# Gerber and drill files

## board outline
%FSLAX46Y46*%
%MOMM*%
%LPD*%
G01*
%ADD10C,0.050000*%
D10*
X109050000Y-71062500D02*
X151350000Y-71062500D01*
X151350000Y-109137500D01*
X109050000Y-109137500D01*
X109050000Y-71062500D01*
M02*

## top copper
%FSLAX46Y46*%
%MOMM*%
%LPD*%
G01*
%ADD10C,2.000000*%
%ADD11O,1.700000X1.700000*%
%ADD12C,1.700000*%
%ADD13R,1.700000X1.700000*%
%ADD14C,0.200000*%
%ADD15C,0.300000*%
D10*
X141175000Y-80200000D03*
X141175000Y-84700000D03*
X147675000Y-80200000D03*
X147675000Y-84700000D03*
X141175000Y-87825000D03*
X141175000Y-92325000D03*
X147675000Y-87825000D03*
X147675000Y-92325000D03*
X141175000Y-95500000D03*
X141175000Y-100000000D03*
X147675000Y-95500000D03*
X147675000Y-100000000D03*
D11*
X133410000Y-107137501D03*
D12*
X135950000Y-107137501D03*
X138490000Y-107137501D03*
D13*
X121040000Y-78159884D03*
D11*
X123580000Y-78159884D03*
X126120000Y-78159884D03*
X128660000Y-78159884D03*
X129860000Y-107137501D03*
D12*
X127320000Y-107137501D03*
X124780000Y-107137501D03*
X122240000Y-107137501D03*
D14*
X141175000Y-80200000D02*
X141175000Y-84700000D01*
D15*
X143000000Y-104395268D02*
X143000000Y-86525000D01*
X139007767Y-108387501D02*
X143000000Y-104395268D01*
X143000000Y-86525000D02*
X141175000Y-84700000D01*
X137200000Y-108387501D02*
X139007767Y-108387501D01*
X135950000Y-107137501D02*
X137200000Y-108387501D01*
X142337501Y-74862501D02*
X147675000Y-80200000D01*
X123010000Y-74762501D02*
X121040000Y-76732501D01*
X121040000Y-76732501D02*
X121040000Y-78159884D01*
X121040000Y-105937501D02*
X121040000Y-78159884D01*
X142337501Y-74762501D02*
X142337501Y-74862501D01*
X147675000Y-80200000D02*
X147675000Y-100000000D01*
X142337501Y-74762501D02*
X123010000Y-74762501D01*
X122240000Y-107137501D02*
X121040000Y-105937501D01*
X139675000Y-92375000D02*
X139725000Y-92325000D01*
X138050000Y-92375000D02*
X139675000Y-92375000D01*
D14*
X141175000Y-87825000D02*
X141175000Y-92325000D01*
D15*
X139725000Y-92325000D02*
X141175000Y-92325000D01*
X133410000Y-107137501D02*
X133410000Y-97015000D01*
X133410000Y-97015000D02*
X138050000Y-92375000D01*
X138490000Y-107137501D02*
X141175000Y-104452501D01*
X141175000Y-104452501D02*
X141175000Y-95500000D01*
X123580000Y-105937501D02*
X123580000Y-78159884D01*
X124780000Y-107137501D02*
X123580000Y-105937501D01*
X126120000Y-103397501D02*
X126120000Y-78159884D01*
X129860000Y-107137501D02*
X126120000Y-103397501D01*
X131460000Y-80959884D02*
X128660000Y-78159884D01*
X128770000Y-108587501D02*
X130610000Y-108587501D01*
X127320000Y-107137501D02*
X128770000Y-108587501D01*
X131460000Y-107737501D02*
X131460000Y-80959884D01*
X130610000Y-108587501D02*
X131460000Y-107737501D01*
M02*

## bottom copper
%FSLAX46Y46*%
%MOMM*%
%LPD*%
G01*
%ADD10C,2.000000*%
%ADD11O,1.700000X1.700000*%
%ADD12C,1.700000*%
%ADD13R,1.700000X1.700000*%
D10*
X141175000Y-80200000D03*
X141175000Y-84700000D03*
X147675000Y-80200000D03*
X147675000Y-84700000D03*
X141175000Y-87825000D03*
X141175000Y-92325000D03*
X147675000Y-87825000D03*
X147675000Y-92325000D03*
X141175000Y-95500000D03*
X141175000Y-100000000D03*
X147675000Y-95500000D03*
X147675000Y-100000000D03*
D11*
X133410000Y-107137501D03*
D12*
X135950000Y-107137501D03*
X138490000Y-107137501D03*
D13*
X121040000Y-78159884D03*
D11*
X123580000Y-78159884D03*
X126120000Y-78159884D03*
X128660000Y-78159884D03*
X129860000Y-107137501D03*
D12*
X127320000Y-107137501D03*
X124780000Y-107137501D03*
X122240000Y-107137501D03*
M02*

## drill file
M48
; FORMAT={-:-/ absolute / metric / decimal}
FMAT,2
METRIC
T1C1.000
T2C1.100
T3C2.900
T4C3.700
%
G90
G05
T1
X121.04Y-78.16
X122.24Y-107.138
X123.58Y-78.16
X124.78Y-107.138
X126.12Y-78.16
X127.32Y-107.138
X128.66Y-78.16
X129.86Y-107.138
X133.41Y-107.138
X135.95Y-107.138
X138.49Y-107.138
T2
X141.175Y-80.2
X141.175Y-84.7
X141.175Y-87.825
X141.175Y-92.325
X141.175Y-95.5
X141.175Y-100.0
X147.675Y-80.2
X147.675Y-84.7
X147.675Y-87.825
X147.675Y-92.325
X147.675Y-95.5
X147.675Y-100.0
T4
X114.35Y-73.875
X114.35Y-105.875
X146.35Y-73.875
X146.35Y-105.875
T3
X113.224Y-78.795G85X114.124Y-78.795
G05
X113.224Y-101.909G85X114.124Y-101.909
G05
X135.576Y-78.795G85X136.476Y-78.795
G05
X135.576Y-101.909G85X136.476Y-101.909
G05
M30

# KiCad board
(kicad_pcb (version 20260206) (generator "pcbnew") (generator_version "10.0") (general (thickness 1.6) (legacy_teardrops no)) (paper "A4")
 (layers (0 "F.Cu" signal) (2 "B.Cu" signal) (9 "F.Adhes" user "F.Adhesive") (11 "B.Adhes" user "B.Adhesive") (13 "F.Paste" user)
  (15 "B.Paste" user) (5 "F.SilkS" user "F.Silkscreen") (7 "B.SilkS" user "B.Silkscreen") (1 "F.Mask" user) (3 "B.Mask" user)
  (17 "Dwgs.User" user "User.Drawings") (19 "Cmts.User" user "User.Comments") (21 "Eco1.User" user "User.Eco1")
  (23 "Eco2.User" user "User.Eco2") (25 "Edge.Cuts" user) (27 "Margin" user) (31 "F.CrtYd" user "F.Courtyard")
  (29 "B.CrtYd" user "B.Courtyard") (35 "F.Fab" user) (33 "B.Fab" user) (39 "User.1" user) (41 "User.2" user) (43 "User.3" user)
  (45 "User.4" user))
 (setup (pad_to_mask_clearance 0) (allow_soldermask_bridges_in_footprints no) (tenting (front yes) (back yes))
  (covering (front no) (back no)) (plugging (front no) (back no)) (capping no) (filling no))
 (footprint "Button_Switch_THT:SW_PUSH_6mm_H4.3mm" (layer "F.Cu") (at 141.175 80.2)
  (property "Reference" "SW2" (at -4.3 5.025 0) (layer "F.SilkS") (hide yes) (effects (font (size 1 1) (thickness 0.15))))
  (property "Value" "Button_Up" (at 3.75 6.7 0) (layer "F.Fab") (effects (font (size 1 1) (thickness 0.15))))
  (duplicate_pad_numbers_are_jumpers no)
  (pad "1" thru_hole circle (at 0 0 90) (size 2 2) (drill 1.1) (layers "*.Cu" "*.Mask") (remove_unused_layers no) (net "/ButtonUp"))
  (pad "1" thru_hole circle (at 0 4.5 90) (size 2 2) (drill 1.1) (layers "*.Cu" "*.Mask") (remove_unused_layers no) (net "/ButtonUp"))
  (pad "2" thru_hole circle (at 6.5 0 90) (size 2 2) (drill 1.1) (layers "*.Cu" "*.Mask") (remove_unused_layers no) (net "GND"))
  (pad "2" thru_hole circle (at 6.5 4.5 90) (size 2 2) (drill 1.1) (layers "*.Cu" "*.Mask") (remove_unused_layers no) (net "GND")))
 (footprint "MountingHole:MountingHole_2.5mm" (layer "F.Cu") (at 146.35 73.875)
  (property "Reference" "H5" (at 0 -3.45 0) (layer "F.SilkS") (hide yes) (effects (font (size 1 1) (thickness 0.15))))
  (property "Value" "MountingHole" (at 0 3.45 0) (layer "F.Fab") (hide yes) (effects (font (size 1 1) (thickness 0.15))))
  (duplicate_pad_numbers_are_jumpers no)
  (pad "" np_thru_hole circle (at 0 0) (size 2.5 2.5) (drill 3.7) (layers "*.Cu" "*.Mask")))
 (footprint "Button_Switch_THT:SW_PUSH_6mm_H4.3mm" (layer "F.Cu") (at 141.175 87.825)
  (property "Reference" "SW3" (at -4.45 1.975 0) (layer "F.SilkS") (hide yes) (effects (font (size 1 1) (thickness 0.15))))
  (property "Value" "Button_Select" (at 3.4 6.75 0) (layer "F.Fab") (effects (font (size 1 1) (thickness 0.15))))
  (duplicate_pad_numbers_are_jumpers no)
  (pad "1" thru_hole circle (at 0 0 90) (size 2 2) (drill 1.1) (layers "*.Cu" "*.Mask") (remove_unused_layers no) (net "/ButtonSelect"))
  (pad "1" thru_hole circle (at 0 4.5 90) (size 2 2) (drill 1.1) (layers "*.Cu" "*.Mask") (remove_unused_layers no) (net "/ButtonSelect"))
  (pad "2" thru_hole circle (at 6.5 0 90) (size 2 2) (drill 1.1) (layers "*.Cu" "*.Mask") (remove_unused_layers no) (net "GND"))
  (pad "2" thru_hole circle (at 6.5 4.5 90) (size 2 2) (drill 1.1) (layers "*.Cu" "*.Mask") (remove_unused_layers no) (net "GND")))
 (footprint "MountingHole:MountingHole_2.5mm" (layer "F.Cu") (at 114.35 105.875)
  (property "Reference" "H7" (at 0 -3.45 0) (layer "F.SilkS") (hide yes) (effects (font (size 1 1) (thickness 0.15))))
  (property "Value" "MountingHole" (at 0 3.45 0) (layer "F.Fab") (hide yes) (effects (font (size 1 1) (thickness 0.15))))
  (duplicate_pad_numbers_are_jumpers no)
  (pad "" np_thru_hole circle (at 0 0) (size 2.5 2.5) (drill 3.7) (layers "*.Cu" "*.Mask")))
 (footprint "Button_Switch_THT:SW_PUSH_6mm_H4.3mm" (layer "F.Cu") (at 141.175 95.5)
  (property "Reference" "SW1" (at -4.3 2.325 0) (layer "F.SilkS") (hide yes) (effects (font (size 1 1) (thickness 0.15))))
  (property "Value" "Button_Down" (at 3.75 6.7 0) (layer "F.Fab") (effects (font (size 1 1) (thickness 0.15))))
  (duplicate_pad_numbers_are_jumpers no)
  (pad "1" thru_hole circle (at 0 0 90) (size 2 2) (drill 1.1) (layers "*.Cu" "*.Mask") (remove_unused_layers no) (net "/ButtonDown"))
  (pad "1" thru_hole circle (at 0 4.5 90) (size 2 2) (drill 1.1) (layers "*.Cu" "*.Mask") (remove_unused_layers no) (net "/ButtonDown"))
  (pad "2" thru_hole circle (at 6.5 0 90) (size 2 2) (drill 1.1) (layers "*.Cu" "*.Mask") (remove_unused_layers no) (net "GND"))
  (pad "2" thru_hole circle (at 6.5 4.5 90) (size 2 2) (drill 1.1) (layers "*.Cu" "*.Mask") (remove_unused_layers no) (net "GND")))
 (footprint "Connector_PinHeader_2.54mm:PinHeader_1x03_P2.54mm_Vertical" (layer "F.Cu") (at 133.41 107.137501 90)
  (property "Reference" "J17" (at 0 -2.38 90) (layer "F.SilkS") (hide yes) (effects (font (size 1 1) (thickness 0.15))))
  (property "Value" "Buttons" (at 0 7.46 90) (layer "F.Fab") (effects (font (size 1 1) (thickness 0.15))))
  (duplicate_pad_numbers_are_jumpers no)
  (pad "1" thru_hole oval (at 0 0 90) (size 1.7 1.7) (drill 1) (layers "*.Cu" "*.Mask") (remove_unused_layers no) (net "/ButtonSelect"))
  (pad "2" thru_hole circle (at 0 2.54 90) (size 1.7 1.7) (drill 1) (layers "*.Cu" "*.Mask") (remove_unused_layers no) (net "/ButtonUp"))
  (pad "3" thru_hole circle (at 0 5.08 90) (size 1.7 1.7) (drill 1) (layers "*.Cu" "*.Mask") (remove_unused_layers no) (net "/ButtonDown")))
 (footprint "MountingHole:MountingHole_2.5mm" (layer "F.Cu") (at 114.35 73.875)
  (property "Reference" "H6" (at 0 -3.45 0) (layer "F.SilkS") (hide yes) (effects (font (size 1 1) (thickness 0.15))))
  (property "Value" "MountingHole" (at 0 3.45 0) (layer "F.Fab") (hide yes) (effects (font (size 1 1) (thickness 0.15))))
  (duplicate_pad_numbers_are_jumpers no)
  (pad "" np_thru_hole circle (at 0 0) (size 2.5 2.5) (drill 3.7) (layers "*.Cu" "*.Mask")))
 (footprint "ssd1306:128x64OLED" (layer "F.Cu") (at 124.85 78.159884)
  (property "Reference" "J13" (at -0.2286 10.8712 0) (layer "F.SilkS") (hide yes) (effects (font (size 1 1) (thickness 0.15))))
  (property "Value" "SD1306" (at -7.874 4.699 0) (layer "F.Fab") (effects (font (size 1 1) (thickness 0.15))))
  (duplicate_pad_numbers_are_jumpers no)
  (pad "" np_thru_hole oval (at -11.176 0.635) (size 3.8 2.9) (drill oval 3.8 2.9) (layers "*.Cu" "*.Mask"))
  (pad "" np_thru_hole oval (at -11.176 23.749) (size 3.8 2.9) (drill oval 3.8 2.9) (layers "*.Cu" "*.Mask"))
  (pad "" np_thru_hole oval (at 11.176 0.635) (size 3.8 2.9) (drill oval 3.8 2.9) (layers "*.Cu" "*.Mask"))
  (pad "" np_thru_hole oval (at 11.176 23.749) (size 3.8 2.9) (drill oval 3.8 2.9) (layers "*.Cu" "*.Mask"))
  (pad "1" thru_hole rect (at -3.81 0 90) (size 1.7 1.7) (drill 1) (layers "*.Cu" "*.Mask") (remove_unused_layers no) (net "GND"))
  (pad "2" thru_hole oval (at -1.27 0 90) (size 1.7 1.7) (drill 1) (layers "*.Cu" "*.Mask") (remove_unused_layers no) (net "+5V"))
  (pad "3" thru_hole oval (at 1.27 0 90) (size 1.7 1.7) (drill 1) (layers "*.Cu" "*.Mask") (remove_unused_layers no) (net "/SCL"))
  (pad "4" thru_hole oval (at 3.81 0 90) (size 1.7 1.7) (drill 1) (layers "*.Cu" "*.Mask") (remove_unused_layers no) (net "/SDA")))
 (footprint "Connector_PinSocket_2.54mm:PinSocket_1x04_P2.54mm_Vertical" (layer "F.Cu") (at 129.86 107.137501 -90)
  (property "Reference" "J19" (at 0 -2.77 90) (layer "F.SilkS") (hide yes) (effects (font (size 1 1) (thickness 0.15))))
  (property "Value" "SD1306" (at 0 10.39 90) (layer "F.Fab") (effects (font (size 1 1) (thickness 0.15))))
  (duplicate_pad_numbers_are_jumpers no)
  (pad "1" thru_hole oval (at 0 0 270) (size 1.7 1.7) (drill 1) (layers "*.Cu" "*.Mask") (remove_unused_layers no) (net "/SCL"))
  (pad "2" thru_hole circle (at 0 2.54 270) (size 1.7 1.7) (drill 1) (layers "*.Cu" "*.Mask") (remove_unused_layers no) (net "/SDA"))
  (pad "3" thru_hole circle (at 0 5.08 270) (size 1.7 1.7) (drill 1) (layers "*.Cu" "*.Mask") (remove_unused_layers no) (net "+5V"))
  (pad "4" thru_hole circle (at 0 7.62 270) (size 1.7 1.7) (drill 1) (layers "*.Cu" "*.Mask") (remove_unused_layers no) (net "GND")))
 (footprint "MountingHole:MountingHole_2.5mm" (layer "F.Cu") (at 146.35 105.875)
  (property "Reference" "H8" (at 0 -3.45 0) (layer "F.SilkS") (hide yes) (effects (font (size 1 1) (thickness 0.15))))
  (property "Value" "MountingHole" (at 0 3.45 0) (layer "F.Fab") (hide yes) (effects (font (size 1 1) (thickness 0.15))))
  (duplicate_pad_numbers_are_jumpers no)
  (pad "" np_thru_hole circle (at 0 0) (size 2.5 2.5) (drill 3.7) (layers "*.Cu" "*.Mask")))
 (gr_rect (start 109.05 71.0625) (end 151.35 109.1375) (stroke (width 0.05) (type solid)) (fill no) (layer "Edge.Cuts"))
 (segment (start 141.175 80.2) (end 141.175 84.7) (width 0.2) (layer "F.Cu") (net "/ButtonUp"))
 (segment (start 143 104.395268) (end 143 86.525) (width 0.3) (layer "F.Cu") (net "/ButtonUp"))
 (segment (start 139.007767 108.387501) (end 143 104.395268) (width 0.3) (layer "F.Cu") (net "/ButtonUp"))
 (segment (start 143 86.525) (end 141.175 84.7) (width 0.3) (layer "F.Cu") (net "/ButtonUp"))
 (segment (start 137.2 108.387501) (end 139.007767 108.387501) (width 0.3) (layer "F.Cu") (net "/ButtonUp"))
 (segment (start 135.95 107.137501) (end 137.2 108.387501) (width 0.3) (layer "F.Cu") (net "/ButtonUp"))
 (segment (start 142.337501 74.862501) (end 147.675 80.2) (width 0.3) (layer "F.Cu") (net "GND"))
 (segment (start 123.01 74.762501) (end 121.04 76.732501) (width 0.3) (layer "F.Cu") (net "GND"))
 (segment (start 121.04 76.732501) (end 121.04 78.159884) (width 0.3) (layer "F.Cu") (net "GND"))
 (segment (start 121.04 105.937501) (end 121.04 78.159884) (width 0.3) (layer "F.Cu") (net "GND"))
 (segment (start 142.337501 74.762501) (end 142.337501 74.862501) (width 0.3) (layer "F.Cu") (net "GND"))
 (segment (start 147.675 80.2) (end 147.675 100) (width 0.3) (layer "F.Cu") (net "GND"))
 (segment (start 142.337501 74.762501) (end 123.01 74.762501) (width 0.3) (layer "F.Cu") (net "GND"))
 (segment (start 122.24 107.137501) (end 121.04 105.937501) (width 0.3) (layer "F.Cu") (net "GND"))
 (segment (start 139.675 92.375) (end 139.725 92.325) (width 0.3) (layer "F.Cu") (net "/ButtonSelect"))
 (segment (start 138.05 92.375) (end 139.675 92.375) (width 0.3) (layer "F.Cu") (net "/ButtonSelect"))
 (segment (start 141.175 87.825) (end 141.175 92.325) (width 0.2) (layer "F.Cu") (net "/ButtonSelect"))
 (segment (start 139.725 92.325) (end 141.175 92.325) (width 0.3) (layer "F.Cu") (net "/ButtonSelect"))
 (segment (start 133.41 107.137501) (end 133.41 97.015) (width 0.3) (layer "F.Cu") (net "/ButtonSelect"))
 (segment (start 133.41 97.015) (end 138.05 92.375) (width 0.3) (layer "F.Cu") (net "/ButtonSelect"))
 (segment (start 138.49 107.137501) (end 141.175 104.452501) (width 0.3) (layer "F.Cu") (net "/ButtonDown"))
 (segment (start 141.175 104.452501) (end 141.175 95.5) (width 0.3) (layer "F.Cu") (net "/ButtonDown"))
 (segment (start 123.58 105.937501) (end 123.58 78.159884) (width 0.3) (layer "F.Cu") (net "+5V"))
 (segment (start 124.78 107.137501) (end 123.58 105.937501) (width 0.3) (layer "F.Cu") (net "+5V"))
 (segment (start 126.12 103.397501) (end 126.12 78.159884) (width 0.3) (layer "F.Cu") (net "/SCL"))
 (segment (start 129.86 107.137501) (end 126.12 103.397501) (width 0.3) (layer "F.Cu") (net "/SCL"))
 (segment (start 131.46 80.959884) (end 128.66 78.159884) (width 0.3) (layer "F.Cu") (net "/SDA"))
 (segment (start 128.77 108.587501) (end 130.61 108.587501) (width 0.3) (layer "F.Cu") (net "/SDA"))
 (segment (start 127.32 107.137501) (end 128.77 108.587501) (width 0.3) (layer "F.Cu") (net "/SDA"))
 (segment (start 131.46 107.737501) (end 131.46 80.959884) (width 0.3) (layer "F.Cu") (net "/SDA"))
 (segment (start 130.61 108.587501) (end 131.46 107.737501) (width 0.3) (layer "F.Cu") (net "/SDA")))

